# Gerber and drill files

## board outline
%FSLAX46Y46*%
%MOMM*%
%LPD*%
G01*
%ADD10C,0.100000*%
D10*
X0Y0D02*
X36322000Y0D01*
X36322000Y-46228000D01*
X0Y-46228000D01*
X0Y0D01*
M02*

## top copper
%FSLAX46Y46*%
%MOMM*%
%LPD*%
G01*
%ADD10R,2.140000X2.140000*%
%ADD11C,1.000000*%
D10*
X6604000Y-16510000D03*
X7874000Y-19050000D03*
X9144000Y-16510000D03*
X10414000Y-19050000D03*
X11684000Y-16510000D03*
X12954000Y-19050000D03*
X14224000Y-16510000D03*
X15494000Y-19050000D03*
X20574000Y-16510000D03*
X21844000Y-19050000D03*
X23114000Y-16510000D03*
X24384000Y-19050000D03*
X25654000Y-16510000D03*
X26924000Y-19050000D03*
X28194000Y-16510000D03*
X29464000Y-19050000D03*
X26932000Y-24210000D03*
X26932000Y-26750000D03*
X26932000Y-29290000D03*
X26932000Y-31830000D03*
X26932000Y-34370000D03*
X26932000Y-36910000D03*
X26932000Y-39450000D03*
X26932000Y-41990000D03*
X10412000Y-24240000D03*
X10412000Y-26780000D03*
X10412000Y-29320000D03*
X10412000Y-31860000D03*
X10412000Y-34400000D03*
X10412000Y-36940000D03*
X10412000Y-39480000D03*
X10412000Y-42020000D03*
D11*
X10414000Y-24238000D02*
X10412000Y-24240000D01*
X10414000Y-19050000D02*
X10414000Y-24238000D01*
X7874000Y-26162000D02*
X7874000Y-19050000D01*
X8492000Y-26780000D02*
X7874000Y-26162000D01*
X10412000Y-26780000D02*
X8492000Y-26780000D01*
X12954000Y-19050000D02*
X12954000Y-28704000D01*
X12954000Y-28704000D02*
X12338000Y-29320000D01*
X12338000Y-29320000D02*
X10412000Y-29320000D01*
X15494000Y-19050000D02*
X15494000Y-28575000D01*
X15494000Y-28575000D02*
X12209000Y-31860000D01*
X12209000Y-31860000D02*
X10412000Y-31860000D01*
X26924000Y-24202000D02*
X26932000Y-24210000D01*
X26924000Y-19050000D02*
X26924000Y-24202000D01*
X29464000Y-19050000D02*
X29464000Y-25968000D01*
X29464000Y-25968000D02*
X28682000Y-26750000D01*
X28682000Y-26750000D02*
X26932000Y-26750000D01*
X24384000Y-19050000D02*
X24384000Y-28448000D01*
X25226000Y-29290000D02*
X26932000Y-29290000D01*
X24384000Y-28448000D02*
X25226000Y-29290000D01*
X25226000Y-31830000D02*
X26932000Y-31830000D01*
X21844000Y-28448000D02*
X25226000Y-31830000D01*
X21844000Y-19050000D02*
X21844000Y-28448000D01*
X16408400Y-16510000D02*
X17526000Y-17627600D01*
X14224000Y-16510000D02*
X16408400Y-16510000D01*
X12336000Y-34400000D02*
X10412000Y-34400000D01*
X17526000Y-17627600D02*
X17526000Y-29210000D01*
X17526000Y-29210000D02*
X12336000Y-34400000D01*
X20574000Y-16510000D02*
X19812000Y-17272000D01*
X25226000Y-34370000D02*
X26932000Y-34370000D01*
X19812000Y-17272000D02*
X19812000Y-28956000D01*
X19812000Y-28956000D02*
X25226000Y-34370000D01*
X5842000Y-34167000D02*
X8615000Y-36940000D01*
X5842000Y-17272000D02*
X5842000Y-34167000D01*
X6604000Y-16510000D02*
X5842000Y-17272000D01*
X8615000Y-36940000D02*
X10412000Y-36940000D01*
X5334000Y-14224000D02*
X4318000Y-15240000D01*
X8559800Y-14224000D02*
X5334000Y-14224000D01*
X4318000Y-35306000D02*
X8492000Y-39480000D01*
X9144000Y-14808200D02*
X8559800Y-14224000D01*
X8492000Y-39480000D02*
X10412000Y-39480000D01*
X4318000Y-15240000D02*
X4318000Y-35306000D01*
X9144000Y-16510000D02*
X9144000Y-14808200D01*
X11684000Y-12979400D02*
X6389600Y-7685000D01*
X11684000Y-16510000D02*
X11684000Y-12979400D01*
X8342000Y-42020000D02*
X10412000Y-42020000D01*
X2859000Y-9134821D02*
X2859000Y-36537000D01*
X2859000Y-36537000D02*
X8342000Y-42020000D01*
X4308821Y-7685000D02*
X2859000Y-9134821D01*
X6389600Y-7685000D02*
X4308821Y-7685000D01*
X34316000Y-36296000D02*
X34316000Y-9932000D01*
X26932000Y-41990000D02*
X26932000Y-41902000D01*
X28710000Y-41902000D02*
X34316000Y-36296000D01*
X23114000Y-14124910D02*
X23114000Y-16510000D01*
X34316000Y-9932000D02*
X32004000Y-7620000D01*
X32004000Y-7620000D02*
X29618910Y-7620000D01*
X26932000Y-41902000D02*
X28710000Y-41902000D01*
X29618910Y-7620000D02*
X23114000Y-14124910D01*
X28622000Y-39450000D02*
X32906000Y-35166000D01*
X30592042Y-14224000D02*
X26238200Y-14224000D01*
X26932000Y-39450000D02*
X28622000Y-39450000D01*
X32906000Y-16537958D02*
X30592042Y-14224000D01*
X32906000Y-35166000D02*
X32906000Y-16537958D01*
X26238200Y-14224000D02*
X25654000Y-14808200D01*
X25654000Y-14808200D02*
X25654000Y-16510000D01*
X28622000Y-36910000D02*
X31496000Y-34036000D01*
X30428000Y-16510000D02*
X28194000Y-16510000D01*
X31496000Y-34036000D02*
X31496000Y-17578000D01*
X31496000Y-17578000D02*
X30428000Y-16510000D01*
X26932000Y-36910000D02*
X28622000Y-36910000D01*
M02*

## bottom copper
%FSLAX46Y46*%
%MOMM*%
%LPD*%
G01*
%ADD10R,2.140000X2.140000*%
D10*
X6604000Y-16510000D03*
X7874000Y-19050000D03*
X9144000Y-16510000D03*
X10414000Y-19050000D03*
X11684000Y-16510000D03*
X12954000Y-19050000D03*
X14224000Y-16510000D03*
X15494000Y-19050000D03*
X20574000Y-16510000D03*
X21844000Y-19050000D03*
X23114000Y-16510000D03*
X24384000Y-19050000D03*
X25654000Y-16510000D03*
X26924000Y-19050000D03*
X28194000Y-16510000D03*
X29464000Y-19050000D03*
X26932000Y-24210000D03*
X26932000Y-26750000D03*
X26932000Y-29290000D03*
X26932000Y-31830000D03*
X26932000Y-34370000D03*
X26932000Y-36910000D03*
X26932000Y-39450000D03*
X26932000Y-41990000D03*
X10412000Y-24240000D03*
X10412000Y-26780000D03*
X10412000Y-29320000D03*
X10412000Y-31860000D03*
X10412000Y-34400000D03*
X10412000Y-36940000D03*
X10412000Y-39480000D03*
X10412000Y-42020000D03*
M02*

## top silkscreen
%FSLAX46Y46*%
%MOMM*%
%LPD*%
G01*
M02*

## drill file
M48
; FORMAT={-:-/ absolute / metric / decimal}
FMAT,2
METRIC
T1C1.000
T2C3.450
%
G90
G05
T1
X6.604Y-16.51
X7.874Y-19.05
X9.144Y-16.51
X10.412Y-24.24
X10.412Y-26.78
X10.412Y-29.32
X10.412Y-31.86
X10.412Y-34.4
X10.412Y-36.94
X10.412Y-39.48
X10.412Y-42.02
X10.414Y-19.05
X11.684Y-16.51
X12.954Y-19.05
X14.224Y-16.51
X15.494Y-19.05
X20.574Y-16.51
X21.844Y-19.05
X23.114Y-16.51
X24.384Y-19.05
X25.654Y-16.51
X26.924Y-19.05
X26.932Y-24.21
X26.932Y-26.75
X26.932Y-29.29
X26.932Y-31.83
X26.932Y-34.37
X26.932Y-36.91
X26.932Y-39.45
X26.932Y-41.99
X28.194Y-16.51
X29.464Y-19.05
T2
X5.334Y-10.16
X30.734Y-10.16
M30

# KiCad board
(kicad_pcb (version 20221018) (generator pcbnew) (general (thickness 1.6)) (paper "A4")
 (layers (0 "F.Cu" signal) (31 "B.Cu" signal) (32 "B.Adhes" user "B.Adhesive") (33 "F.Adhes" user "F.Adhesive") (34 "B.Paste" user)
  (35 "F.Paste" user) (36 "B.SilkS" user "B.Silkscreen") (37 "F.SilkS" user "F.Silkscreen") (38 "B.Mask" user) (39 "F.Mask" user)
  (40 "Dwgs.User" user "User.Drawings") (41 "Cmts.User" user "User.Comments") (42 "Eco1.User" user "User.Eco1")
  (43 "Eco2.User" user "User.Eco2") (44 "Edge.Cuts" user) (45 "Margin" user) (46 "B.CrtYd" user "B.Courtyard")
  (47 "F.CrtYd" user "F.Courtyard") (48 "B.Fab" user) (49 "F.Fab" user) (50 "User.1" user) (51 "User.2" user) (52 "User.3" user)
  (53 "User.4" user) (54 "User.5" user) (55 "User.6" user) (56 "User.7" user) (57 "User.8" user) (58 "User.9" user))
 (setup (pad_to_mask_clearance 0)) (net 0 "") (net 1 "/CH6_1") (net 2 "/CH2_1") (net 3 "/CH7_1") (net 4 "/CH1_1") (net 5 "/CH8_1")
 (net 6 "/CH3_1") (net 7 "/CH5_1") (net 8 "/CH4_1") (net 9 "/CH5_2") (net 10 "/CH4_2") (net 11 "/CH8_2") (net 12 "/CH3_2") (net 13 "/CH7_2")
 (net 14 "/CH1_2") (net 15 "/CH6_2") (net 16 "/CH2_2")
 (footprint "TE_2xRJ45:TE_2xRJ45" (layer "B.Cu") (at 18.034 10.435)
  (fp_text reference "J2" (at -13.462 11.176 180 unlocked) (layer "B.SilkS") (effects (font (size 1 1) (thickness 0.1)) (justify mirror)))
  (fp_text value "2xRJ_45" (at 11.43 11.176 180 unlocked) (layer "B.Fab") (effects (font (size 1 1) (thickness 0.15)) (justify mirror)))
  (pad "" np_thru_hole circle (at -12.7 -0.275) (size 3.25 3.25) (drill 3.45) (layers "F&B.Cu" "*.Mask"))
  (pad "" np_thru_hole circle (at 12.7 -0.275) (size 3.45 3.45) (drill 3.45) (layers "F&B.Cu" "*.Mask"))
  (pad "1_1" thru_hole rect (at -11.43 6.075) (size 2.14 2.14) (drill 1) (layers "*.Cu" "*.Mask") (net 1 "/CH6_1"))
  (pad "1_2" thru_hole rect (at -10.16 8.615) (size 2.14 2.14) (drill 1) (layers "*.Cu" "*.Mask") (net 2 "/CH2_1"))
  (pad "1_3" thru_hole rect (at -8.89 6.075) (size 2.14 2.14) (drill 1) (layers "*.Cu" "*.Mask") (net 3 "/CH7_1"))
  (pad "1_4" thru_hole rect (at -7.62 8.615) (size 2.14 2.14) (drill 1) (layers "*.Cu" "*.Mask") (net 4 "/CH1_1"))
  (pad "1_5" thru_hole rect (at -6.35 6.075) (size 2.14 2.14) (drill 1) (layers "*.Cu" "*.Mask") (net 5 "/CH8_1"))
  (pad "1_6" thru_hole rect (at -5.08 8.615) (size 2.14 2.14) (drill 1) (layers "*.Cu" "*.Mask") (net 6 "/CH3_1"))
  (pad "1_7" thru_hole rect (at -3.81 6.075) (size 2.14 2.14) (drill 1) (layers "*.Cu" "*.Mask") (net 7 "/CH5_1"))
  (pad "1_8" thru_hole rect (at -2.54 8.615) (size 2.14 2.14) (drill 1) (layers "*.Cu" "*.Mask") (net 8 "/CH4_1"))
  (pad "2_1" thru_hole rect (at 2.54 6.075) (size 2.14 2.14) (drill 1) (layers "*.Cu" "*.Mask") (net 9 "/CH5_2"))
  (pad "2_2" thru_hole rect (at 3.81 8.615) (size 2.14 2.14) (drill 1) (layers "*.Cu" "*.Mask") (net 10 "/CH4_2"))
  (pad "2_3" thru_hole rect (at 5.08 6.075) (size 2.14 2.14) (drill 1) (layers "*.Cu" "*.Mask") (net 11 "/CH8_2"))
  (pad "2_4" thru_hole rect (at 6.35 8.615) (size 2.14 2.14) (drill 1) (layers "*.Cu" "*.Mask") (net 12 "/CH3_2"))
  (pad "2_5" thru_hole rect (at 7.62 6.075) (size 2.14 2.14) (drill 1) (layers "*.Cu" "*.Mask") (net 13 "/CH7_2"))
  (pad "2_6" thru_hole rect (at 8.89 8.615) (size 2.14 2.14) (drill 1) (layers "*.Cu" "*.Mask") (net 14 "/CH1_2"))
  (pad "2_7" thru_hole rect (at 10.16 6.075) (size 2.14 2.14) (drill 1) (layers "*.Cu" "*.Mask") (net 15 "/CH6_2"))
  (pad "2_8" thru_hole rect (at 11.43 8.615) (size 2.14 2.14) (drill 1) (layers "*.Cu" "*.Mask") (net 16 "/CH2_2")))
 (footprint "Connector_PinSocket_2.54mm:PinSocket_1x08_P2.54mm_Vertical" (layer "B.Cu") (at 26.932 24.21 180)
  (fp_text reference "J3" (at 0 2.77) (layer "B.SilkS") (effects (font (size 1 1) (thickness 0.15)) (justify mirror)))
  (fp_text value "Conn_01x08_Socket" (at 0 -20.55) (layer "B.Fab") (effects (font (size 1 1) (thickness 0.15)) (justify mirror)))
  (pad "1" thru_hole rect (at 0 0 180) (size 2.14 2.14) (drill 1) (layers "*.Cu" "*.Mask") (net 14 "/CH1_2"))
  (pad "2" thru_hole rect (at 0 -2.54 180) (size 2.14 2.14) (drill 1) (layers "*.Cu" "*.Mask") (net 16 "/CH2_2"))
  (pad "3" thru_hole rect (at 0 -5.08 180) (size 2.14 2.14) (drill 1) (layers "*.Cu" "*.Mask") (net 12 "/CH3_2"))
  (pad "4" thru_hole rect (at 0 -7.62 180) (size 2.14 2.14) (drill 1) (layers "*.Cu" "*.Mask") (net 10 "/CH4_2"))
  (pad "5" thru_hole rect (at 0 -10.16 180) (size 2.14 2.14) (drill 1) (layers "*.Cu" "*.Mask") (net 9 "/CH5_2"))
  (pad "6" thru_hole rect (at 0 -12.7 180) (size 2.14 2.14) (drill 1) (layers "*.Cu" "*.Mask") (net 15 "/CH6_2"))
  (pad "7" thru_hole rect (at 0 -15.24 180) (size 2.14 2.14) (drill 1) (layers "*.Cu" "*.Mask") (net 13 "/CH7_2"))
  (pad "8" thru_hole rect (at 0 -17.78 180) (size 2.14 2.14) (drill 1) (layers "*.Cu" "*.Mask") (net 11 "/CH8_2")))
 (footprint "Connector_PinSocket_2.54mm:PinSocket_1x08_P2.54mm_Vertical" (layer "B.Cu") (at 10.412 24.24 180)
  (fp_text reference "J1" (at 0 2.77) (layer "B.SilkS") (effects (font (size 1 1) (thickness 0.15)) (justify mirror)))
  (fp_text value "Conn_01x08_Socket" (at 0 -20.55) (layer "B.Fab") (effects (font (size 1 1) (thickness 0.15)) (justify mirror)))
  (pad "1" thru_hole rect (at 0 0 180) (size 2.14 2.14) (drill 1) (layers "*.Cu" "*.Mask") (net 4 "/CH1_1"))
  (pad "2" thru_hole rect (at 0 -2.54 180) (size 2.14 2.14) (drill 1) (layers "*.Cu" "*.Mask") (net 2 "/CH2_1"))
  (pad "3" thru_hole rect (at 0 -5.08 180) (size 2.14 2.14) (drill 1) (layers "*.Cu" "*.Mask") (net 6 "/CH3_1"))
  (pad "4" thru_hole rect (at 0 -7.62 180) (size 2.14 2.14) (drill 1) (layers "*.Cu" "*.Mask") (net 8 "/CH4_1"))
  (pad "5" thru_hole rect (at 0 -10.16 180) (size 2.14 2.14) (drill 1) (layers "*.Cu" "*.Mask") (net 7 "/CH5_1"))
  (pad "6" thru_hole rect (at 0 -12.7 180) (size 2.14 2.14) (drill 1) (layers "*.Cu" "*.Mask") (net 1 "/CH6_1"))
  (pad "7" thru_hole rect (at 0 -15.24 180) (size 2.14 2.14) (drill 1) (layers "*.Cu" "*.Mask") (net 3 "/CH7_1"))
  (pad "8" thru_hole rect (at 0 -17.78 180) (size 2.14 2.14) (drill 1) (layers "*.Cu" "*.Mask") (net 5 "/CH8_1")))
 (gr_rect (start 0 0) (end 36.322 46.228) (stroke (width 0.1) (type default)) (fill none) (layer "Edge.Cuts"))
 (segment (start 10.414 24.238) (end 10.412 24.24) (width 1) (layer "F.Cu") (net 4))
 (segment (start 10.414 19.05) (end 10.414 24.238) (width 1) (layer "F.Cu") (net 4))
 (segment (start 7.874 26.162) (end 7.874 19.05) (width 1) (layer "F.Cu") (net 2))
 (segment (start 8.492 26.78) (end 7.874 26.162) (width 1) (layer "F.Cu") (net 2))
 (segment (start 10.412 26.78) (end 8.492 26.78) (width 1) (layer "F.Cu") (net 2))
 (segment (start 12.954 19.05) (end 12.954 28.704) (width 1) (layer "F.Cu") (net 6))
 (segment (start 12.954 28.704) (end 12.338 29.32) (width 1) (layer "F.Cu") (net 6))
 (segment (start 12.338 29.32) (end 10.412 29.32) (width 1) (layer "F.Cu") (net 6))
 (segment (start 15.494 19.05) (end 15.494 28.575) (width 1) (layer "F.Cu") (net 8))
 (segment (start 15.494 28.575) (end 12.209 31.86) (width 1) (layer "F.Cu") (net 8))
 (segment (start 12.209 31.86) (end 10.412 31.86) (width 1) (layer "F.Cu") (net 8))
 (segment (start 26.924 24.202) (end 26.932 24.21) (width 1) (layer "F.Cu") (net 14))
 (segment (start 26.924 19.05) (end 26.924 24.202) (width 1) (layer "F.Cu") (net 14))
 (segment (start 29.464 19.05) (end 29.464 25.968) (width 1) (layer "F.Cu") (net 16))
 (segment (start 29.464 25.968) (end 28.682 26.75) (width 1) (layer "F.Cu") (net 16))
 (segment (start 28.682 26.75) (end 26.932 26.75) (width 1) (layer "F.Cu") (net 16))
 (segment (start 24.384 19.05) (end 24.384 28.448) (width 1) (layer "F.Cu") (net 12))
 (segment (start 25.226 29.29) (end 26.932 29.29) (width 1) (layer "F.Cu") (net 12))
 (segment (start 24.384 28.448) (end 25.226 29.29) (width 1) (layer "F.Cu") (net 12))
 (segment (start 25.226 31.83) (end 26.932 31.83) (width 1) (layer "F.Cu") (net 10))
 (segment (start 21.844 28.448) (end 25.226 31.83) (width 1) (layer "F.Cu") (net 10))
 (segment (start 21.844 19.05) (end 21.844 28.448) (width 1) (layer "F.Cu") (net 10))
 (segment (start 16.4084 16.51) (end 17.526 17.6276) (width 1) (layer "F.Cu") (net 7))
 (segment (start 14.224 16.51) (end 16.4084 16.51) (width 1) (layer "F.Cu") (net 7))
 (segment (start 12.336 34.4) (end 10.412 34.4) (width 1) (layer "F.Cu") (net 7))
 (segment (start 17.526 17.6276) (end 17.526 29.21) (width 1) (layer "F.Cu") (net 7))
 (segment (start 17.526 29.21) (end 12.336 34.4) (width 1) (layer "F.Cu") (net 7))
 (segment (start 20.574 16.51) (end 19.812 17.272) (width 1) (layer "F.Cu") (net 9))
 (segment (start 25.226 34.37) (end 26.932 34.37) (width 1) (layer "F.Cu") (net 9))
 (segment (start 19.812 17.272) (end 19.812 28.956) (width 1) (layer "F.Cu") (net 9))
 (segment (start 19.812 28.956) (end 25.226 34.37) (width 1) (layer "F.Cu") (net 9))
 (segment (start 5.842 34.167) (end 8.615 36.94) (width 1) (layer "F.Cu") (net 1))
 (segment (start 5.842 17.272) (end 5.842 34.167) (width 1) (layer "F.Cu") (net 1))
 (segment (start 6.604 16.51) (end 5.842 17.272) (width 1) (layer "F.Cu") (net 1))
 (segment (start 8.615 36.94) (end 10.412 36.94) (width 1) (layer "F.Cu") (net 1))
 (segment (start 5.334 14.224) (end 4.318 15.24) (width 1) (layer "F.Cu") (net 3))
 (segment (start 8.5598 14.224) (end 5.334 14.224) (width 1) (layer "F.Cu") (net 3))
 (segment (start 4.318 35.306) (end 8.492 39.48) (width 1) (layer "F.Cu") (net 3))
 (segment (start 9.144 14.8082) (end 8.5598 14.224) (width 1) (layer "F.Cu") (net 3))
 (segment (start 8.492 39.48) (end 10.412 39.48) (width 1) (layer "F.Cu") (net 3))
 (segment (start 4.318 15.24) (end 4.318 35.306) (width 1) (layer "F.Cu") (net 3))
 (segment (start 9.144 16.51) (end 9.144 14.8082) (width 1) (layer "F.Cu") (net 3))
 (segment (start 11.684 12.9794) (end 6.3896 7.685) (width 1) (layer "F.Cu") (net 5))
 (segment (start 11.684 16.51) (end 11.684 12.9794) (width 1) (layer "F.Cu") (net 5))
 (segment (start 8.342 42.02) (end 10.412 42.02) (width 1) (layer "F.Cu") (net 5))
 (segment (start 2.859 9.134821) (end 2.859 36.537) (width 1) (layer "F.Cu") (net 5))
 (segment (start 2.859 36.537) (end 8.342 42.02) (width 1) (layer "F.Cu") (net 5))
 (segment (start 4.308821 7.685) (end 2.859 9.134821) (width 1) (layer "F.Cu") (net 5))
 (segment (start 6.3896 7.685) (end 4.308821 7.685) (width 1) (layer "F.Cu") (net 5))
 (segment (start 34.316 36.296) (end 34.316 9.932) (width 1) (layer "F.Cu") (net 11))
 (segment (start 26.932 41.99) (end 26.932 41.902) (width 1) (layer "F.Cu") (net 11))
 (segment (start 28.71 41.902) (end 34.316 36.296) (width 1) (layer "F.Cu") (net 11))
 (segment (start 23.114 14.12491) (end 23.114 16.51) (width 1) (layer "F.Cu") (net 11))
 (segment (start 34.316 9.932) (end 32.004 7.62) (width 1) (layer "F.Cu") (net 11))
 (segment (start 32.004 7.62) (end 29.61891 7.62) (width 1) (layer "F.Cu") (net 11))
 (segment (start 26.932 41.902) (end 28.71 41.902) (width 1) (layer "F.Cu") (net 11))
 (segment (start 29.61891 7.62) (end 23.114 14.12491) (width 1) (layer "F.Cu") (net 11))
 (segment (start 28.622 39.45) (end 32.906 35.166) (width 1) (layer "F.Cu") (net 13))
 (segment (start 30.592042 14.224) (end 26.2382 14.224) (width 1) (layer "F.Cu") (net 13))
 (segment (start 26.932 39.45) (end 28.622 39.45) (width 1) (layer "F.Cu") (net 13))
 (segment (start 32.906 16.537958) (end 30.592042 14.224) (width 1) (layer "F.Cu") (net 13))
 (segment (start 32.906 35.166) (end 32.906 16.537958) (width 1) (layer "F.Cu") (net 13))
 (segment (start 26.2382 14.224) (end 25.654 14.8082) (width 1) (layer "F.Cu") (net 13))
 (segment (start 25.654 14.8082) (end 25.654 16.51) (width 1) (layer "F.Cu") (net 13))
 (segment (start 28.622 36.91) (end 31.496 34.036) (width 1) (layer "F.Cu") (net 15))
 (segment (start 30.428 16.51) (end 28.194 16.51) (width 1) (layer "F.Cu") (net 15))
 (segment (start 31.496 34.036) (end 31.496 17.578) (width 1) (layer "F.Cu") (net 15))
 (segment (start 31.496 17.578) (end 30.428 16.51) (width 1) (layer "F.Cu") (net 15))
 (segment (start 26.932 36.91) (end 28.622 36.91) (width 1) (layer "F.Cu") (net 15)))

